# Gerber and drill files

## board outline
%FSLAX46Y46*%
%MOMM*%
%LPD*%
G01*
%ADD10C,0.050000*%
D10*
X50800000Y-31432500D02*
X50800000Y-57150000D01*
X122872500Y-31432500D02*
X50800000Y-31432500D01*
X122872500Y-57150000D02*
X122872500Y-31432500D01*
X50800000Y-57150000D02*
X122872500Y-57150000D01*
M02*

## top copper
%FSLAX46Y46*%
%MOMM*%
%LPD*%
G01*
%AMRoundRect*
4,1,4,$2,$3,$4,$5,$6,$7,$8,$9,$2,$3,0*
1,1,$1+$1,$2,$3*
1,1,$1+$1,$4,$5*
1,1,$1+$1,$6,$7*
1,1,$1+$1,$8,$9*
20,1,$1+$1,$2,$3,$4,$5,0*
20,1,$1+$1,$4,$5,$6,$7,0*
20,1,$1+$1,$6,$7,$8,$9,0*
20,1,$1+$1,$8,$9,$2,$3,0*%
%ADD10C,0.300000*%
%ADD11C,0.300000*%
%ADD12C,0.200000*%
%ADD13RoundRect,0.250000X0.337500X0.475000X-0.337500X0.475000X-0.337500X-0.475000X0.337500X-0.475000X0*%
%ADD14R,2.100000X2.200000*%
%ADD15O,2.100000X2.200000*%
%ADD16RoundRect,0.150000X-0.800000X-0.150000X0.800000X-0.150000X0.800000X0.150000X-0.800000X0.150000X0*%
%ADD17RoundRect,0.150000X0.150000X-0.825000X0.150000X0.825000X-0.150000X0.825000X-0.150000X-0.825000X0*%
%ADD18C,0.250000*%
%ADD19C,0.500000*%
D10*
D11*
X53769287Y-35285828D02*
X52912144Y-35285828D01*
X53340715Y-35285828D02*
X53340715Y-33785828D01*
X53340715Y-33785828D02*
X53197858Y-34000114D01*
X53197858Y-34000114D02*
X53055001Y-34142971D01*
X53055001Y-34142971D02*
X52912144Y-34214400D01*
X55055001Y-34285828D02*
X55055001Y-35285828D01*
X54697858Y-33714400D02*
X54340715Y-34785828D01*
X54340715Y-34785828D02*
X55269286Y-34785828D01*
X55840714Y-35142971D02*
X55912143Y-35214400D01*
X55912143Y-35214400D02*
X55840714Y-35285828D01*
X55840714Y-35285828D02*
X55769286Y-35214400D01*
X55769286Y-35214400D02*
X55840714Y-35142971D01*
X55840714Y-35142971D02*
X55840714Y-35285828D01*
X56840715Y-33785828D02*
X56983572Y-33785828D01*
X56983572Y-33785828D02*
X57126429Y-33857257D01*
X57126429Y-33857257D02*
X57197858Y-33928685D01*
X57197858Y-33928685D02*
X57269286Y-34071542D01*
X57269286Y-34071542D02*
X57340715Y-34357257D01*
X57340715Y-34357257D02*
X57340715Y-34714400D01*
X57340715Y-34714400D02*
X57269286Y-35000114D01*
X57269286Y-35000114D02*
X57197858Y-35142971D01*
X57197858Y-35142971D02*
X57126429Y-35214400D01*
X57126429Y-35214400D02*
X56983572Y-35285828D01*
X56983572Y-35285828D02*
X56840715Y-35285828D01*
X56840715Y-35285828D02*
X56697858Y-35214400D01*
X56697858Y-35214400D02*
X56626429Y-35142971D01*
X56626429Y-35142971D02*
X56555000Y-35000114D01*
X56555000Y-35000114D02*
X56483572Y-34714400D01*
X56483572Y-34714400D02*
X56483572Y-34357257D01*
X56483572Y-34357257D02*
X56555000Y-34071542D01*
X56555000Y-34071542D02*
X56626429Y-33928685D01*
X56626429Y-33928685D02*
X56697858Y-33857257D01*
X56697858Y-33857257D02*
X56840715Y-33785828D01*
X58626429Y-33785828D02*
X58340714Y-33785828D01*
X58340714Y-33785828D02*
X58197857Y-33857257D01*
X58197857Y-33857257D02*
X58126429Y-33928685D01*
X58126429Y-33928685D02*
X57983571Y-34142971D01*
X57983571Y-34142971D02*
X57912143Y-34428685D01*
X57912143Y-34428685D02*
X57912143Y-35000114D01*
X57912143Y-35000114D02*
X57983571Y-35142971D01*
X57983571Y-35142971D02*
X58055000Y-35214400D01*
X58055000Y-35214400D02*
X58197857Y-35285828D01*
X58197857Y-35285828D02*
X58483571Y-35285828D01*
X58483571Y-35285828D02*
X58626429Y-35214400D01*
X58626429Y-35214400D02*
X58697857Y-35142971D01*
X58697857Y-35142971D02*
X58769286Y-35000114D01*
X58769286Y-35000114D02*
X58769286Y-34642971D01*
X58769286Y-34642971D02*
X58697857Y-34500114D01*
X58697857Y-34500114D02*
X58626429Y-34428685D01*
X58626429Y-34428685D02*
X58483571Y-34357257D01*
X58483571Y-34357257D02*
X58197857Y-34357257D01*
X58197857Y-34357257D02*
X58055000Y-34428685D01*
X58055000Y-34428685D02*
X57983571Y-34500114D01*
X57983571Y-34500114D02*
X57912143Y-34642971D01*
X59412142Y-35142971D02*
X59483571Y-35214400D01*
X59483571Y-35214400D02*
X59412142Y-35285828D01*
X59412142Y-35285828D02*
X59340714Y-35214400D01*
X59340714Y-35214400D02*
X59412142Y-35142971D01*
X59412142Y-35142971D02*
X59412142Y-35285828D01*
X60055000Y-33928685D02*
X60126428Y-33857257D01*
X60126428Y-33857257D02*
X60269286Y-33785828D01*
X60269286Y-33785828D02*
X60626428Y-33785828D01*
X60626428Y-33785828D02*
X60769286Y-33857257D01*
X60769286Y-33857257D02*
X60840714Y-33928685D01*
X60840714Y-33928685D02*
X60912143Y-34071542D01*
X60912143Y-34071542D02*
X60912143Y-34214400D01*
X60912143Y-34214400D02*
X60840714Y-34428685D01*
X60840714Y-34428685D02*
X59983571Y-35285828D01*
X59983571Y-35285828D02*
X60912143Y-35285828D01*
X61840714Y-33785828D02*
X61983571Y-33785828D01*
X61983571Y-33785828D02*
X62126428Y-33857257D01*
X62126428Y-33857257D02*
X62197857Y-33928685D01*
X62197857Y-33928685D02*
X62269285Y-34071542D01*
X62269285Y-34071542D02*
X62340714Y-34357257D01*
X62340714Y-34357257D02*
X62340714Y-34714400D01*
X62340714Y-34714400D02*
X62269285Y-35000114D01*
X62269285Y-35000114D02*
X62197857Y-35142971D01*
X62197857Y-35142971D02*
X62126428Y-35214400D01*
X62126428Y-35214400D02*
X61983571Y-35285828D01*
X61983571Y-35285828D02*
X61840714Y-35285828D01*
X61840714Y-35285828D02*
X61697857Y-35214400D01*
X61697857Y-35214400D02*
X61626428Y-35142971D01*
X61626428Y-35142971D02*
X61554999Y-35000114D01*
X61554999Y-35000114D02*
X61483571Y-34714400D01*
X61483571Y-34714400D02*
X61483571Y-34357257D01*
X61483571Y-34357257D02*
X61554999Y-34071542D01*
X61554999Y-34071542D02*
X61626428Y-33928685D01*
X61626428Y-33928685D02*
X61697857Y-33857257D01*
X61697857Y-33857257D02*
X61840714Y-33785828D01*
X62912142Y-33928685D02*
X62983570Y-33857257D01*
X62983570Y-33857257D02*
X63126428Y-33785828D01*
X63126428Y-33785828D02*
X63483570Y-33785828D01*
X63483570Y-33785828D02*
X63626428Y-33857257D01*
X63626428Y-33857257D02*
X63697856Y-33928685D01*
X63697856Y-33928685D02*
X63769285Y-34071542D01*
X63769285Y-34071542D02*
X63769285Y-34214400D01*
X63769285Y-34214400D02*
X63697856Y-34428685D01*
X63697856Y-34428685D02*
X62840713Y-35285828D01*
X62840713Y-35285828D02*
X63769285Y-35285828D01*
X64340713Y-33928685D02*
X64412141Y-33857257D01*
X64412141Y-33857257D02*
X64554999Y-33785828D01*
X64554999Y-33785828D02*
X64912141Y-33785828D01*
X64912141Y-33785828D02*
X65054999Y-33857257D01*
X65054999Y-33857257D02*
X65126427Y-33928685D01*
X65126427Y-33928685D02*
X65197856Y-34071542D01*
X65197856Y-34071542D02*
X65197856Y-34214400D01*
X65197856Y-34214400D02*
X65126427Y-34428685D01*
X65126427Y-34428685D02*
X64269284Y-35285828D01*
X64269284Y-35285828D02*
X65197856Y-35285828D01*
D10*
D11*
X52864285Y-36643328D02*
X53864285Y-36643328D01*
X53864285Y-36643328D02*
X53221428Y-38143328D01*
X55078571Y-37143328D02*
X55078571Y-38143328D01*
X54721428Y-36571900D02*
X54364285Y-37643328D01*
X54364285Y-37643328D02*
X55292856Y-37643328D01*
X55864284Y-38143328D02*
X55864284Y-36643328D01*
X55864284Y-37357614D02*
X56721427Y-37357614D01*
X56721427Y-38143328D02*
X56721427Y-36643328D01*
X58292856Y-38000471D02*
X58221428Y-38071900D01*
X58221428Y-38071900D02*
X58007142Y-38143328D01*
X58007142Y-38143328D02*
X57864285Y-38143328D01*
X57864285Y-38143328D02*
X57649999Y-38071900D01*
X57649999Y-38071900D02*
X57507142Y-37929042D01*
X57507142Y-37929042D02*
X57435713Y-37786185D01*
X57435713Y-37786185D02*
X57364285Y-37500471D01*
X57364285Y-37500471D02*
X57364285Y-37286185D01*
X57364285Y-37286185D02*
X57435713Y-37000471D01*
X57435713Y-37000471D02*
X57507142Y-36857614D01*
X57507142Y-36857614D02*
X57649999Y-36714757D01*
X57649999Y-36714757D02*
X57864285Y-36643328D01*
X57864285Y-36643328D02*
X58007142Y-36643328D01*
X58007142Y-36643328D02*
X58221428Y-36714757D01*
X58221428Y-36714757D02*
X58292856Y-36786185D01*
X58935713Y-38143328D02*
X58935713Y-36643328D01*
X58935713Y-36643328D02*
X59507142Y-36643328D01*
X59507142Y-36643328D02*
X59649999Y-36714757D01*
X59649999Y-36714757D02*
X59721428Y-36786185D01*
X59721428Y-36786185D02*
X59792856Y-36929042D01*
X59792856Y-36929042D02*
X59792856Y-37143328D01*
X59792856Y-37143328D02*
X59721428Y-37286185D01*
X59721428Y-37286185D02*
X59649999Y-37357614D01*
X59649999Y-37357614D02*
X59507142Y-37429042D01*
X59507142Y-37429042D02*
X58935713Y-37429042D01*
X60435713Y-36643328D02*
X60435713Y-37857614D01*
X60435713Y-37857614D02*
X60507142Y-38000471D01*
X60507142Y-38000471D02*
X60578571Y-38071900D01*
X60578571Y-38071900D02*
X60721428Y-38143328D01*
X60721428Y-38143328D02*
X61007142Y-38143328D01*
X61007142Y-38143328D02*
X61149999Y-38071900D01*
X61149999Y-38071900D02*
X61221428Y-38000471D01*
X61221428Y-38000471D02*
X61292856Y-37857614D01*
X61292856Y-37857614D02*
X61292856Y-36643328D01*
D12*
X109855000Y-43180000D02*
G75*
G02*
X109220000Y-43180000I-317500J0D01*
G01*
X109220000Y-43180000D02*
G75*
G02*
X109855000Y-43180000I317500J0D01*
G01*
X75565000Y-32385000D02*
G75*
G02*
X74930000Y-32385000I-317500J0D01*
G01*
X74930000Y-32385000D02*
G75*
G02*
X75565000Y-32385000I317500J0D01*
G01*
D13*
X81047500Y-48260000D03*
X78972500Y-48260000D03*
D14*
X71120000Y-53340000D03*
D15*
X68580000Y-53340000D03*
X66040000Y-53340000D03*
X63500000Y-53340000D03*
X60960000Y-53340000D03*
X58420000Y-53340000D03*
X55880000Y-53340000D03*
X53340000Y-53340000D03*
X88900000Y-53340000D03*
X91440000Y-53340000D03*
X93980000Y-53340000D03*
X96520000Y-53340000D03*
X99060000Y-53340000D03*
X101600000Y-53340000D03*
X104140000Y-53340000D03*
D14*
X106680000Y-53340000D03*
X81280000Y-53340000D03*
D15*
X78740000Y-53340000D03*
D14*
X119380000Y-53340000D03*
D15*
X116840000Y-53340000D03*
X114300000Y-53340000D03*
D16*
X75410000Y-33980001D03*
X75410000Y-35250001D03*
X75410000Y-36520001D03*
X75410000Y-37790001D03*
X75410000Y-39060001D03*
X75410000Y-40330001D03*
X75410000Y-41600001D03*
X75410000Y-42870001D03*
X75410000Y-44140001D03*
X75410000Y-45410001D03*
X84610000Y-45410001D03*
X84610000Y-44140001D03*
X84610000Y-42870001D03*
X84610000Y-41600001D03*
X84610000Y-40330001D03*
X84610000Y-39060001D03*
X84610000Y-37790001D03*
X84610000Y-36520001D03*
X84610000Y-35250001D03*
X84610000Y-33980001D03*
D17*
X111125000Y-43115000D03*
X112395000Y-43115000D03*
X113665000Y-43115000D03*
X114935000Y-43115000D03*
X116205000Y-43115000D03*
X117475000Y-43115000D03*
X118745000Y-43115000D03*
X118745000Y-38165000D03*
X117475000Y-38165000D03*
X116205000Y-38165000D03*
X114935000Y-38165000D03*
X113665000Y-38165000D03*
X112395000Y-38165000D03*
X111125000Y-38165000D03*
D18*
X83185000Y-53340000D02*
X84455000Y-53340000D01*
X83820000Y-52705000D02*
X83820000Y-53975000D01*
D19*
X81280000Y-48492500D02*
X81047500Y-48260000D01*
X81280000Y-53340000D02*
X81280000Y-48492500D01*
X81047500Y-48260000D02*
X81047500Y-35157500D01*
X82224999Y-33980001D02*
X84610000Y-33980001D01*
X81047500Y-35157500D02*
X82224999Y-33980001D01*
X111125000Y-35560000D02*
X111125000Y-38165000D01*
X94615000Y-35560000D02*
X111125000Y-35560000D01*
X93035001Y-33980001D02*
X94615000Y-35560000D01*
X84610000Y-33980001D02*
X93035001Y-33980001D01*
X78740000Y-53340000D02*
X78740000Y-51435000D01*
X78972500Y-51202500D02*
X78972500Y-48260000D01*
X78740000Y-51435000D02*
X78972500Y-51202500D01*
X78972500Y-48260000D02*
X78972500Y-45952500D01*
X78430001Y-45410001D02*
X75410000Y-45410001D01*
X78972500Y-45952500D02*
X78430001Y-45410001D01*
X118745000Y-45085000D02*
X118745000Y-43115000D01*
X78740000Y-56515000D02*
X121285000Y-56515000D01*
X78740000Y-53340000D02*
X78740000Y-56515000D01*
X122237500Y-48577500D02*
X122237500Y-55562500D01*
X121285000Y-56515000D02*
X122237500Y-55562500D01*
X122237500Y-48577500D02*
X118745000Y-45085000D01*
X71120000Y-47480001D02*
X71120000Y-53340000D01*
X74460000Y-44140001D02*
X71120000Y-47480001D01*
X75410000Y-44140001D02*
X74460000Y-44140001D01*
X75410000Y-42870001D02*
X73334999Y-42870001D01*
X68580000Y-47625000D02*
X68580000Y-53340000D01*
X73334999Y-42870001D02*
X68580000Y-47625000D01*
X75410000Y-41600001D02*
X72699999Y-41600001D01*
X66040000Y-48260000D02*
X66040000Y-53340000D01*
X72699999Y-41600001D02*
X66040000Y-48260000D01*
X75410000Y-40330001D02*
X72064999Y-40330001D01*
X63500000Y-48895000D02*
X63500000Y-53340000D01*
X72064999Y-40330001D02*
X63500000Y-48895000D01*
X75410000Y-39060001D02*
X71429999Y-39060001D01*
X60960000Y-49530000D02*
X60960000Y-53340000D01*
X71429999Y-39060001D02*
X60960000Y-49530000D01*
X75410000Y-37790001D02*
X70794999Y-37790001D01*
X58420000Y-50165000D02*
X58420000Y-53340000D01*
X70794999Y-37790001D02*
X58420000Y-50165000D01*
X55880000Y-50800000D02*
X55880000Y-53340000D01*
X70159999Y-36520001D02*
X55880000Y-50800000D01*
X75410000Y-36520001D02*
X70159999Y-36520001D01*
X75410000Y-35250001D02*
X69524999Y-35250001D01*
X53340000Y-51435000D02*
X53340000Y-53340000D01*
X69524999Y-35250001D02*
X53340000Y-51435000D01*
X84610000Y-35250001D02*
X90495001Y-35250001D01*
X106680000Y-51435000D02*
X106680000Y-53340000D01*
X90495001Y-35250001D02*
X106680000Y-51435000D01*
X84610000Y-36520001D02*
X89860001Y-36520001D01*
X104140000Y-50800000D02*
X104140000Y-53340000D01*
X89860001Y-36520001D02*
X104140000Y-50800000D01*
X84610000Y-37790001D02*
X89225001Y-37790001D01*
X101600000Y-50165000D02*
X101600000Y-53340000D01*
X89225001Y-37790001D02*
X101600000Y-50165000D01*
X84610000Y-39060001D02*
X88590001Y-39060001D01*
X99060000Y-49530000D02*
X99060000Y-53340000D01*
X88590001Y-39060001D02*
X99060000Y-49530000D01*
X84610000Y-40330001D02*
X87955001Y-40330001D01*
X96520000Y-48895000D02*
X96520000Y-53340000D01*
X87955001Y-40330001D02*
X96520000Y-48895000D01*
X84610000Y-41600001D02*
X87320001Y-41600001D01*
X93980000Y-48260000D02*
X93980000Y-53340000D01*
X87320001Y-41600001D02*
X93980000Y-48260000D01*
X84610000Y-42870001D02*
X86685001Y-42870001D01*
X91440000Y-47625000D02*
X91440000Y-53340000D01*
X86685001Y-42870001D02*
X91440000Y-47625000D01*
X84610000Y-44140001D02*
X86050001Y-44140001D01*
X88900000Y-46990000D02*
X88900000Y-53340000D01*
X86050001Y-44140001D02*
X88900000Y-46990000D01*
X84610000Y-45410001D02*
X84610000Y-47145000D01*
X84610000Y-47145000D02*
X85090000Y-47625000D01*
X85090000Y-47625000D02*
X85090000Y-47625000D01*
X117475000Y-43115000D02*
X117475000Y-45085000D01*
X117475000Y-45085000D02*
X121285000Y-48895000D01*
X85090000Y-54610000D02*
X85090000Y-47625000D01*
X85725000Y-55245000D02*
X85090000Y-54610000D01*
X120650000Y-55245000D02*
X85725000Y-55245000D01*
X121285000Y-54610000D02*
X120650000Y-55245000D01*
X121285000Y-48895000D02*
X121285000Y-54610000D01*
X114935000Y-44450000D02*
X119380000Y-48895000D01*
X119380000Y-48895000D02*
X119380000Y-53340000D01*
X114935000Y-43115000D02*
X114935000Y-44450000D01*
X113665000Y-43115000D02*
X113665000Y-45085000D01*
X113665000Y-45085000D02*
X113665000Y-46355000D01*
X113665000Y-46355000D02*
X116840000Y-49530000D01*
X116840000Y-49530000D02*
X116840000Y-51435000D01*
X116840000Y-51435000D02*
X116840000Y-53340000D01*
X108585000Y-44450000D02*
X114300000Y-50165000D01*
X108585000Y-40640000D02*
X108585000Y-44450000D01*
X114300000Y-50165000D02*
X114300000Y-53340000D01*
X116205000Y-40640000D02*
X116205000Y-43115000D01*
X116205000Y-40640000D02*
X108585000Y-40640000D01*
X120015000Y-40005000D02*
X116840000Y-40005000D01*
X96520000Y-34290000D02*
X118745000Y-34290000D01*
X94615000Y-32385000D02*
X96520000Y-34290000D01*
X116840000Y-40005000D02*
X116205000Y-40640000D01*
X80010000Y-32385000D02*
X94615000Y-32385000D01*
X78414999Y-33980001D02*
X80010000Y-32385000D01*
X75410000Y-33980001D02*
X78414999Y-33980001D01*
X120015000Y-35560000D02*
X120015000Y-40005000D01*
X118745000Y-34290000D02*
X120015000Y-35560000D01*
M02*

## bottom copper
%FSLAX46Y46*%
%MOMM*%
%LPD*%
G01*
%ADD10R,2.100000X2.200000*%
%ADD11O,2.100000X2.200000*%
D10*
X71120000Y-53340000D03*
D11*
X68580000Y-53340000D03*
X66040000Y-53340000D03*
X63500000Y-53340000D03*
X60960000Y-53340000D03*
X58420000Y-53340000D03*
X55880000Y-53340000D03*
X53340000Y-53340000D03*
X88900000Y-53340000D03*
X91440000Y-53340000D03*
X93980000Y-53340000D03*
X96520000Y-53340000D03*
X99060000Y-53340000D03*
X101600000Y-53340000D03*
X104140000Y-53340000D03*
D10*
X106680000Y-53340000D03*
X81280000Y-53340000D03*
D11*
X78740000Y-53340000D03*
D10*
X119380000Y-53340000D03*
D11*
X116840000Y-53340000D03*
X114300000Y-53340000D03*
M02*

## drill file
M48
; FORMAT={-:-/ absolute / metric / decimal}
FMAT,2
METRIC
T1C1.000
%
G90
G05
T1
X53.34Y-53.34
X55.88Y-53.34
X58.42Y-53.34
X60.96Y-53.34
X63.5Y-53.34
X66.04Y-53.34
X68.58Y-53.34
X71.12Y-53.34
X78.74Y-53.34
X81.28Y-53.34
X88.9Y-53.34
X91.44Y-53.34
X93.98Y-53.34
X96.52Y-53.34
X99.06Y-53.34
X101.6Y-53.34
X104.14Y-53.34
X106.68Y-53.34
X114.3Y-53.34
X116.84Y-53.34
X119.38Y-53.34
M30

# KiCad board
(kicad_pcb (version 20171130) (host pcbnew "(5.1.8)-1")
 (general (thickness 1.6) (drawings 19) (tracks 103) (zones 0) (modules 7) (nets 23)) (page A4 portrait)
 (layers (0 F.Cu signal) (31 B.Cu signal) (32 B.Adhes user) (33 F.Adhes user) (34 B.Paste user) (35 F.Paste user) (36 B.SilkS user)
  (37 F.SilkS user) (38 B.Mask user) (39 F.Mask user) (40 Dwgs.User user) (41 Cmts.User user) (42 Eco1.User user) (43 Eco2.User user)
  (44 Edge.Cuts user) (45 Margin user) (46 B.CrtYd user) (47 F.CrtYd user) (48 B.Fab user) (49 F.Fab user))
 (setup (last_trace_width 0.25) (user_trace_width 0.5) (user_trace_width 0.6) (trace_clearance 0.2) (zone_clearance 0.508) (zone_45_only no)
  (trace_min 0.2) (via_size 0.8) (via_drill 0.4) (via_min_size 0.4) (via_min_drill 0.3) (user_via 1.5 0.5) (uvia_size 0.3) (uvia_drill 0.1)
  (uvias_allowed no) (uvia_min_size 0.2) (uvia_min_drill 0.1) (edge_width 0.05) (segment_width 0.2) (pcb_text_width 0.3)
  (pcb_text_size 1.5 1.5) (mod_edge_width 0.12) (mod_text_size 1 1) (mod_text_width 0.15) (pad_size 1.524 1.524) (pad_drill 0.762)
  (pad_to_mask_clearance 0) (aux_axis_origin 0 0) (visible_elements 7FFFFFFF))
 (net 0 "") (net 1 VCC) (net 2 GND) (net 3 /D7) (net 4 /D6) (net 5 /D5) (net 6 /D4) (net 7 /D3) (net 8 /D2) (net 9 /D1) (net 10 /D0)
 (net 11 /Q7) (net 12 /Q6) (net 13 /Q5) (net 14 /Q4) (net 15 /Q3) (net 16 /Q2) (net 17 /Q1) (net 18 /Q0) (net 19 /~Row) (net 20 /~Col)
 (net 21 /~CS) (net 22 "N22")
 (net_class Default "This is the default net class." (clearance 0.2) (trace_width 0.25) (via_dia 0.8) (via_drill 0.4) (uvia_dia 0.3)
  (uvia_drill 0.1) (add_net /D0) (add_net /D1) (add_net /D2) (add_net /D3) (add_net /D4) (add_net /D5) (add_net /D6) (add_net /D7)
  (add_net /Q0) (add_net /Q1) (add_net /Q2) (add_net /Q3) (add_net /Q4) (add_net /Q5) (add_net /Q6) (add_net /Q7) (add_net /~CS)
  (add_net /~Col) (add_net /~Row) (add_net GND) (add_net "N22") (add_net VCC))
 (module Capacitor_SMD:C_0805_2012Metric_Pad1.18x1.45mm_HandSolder (layer F.Cu) (at 80.01 48.26 180)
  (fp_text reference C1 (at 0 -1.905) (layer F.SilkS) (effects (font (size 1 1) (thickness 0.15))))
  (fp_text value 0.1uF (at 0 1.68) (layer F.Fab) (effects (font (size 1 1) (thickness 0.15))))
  (pad 1 smd roundrect (at -1.0375 0 180) (size 1.175 1.45) (layers F.Cu F.Paste F.Mask) (roundrect_rratio 0.2127659574468085) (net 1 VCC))
  (pad 2 smd roundrect (at 1.0375 0 180) (size 1.175 1.45) (layers F.Cu F.Paste F.Mask) (roundrect_rratio 0.2127659574468085) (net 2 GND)))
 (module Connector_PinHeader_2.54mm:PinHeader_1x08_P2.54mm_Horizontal (layer F.Cu) (at 71.12 53.34 270)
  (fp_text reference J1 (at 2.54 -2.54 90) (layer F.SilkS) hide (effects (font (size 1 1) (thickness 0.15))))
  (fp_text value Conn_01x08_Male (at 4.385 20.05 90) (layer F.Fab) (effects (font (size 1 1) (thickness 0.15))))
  (pad 1 thru_hole rect (at 0 0 270) (size 2.2 2.1) (drill 1) (layers *.Cu *.Mask) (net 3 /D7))
  (pad 2 thru_hole oval (at 0 2.54 270) (size 2.2 2.1) (drill 1) (layers *.Cu *.Mask) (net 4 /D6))
  (pad 3 thru_hole oval (at 0 5.08 270) (size 2.2 2.1) (drill 1) (layers *.Cu *.Mask) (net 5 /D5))
  (pad 4 thru_hole oval (at 0 7.62 270) (size 2.2 2.1) (drill 1) (layers *.Cu *.Mask) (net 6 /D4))
  (pad 5 thru_hole oval (at 0 10.16 270) (size 2.2 2.1) (drill 1) (layers *.Cu *.Mask) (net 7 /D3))
  (pad 6 thru_hole oval (at 0 12.7 270) (size 2.2 2.1) (drill 1) (layers *.Cu *.Mask) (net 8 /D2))
  (pad 7 thru_hole oval (at 0 15.24 270) (size 2.2 2.1) (drill 1) (layers *.Cu *.Mask) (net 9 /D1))
  (pad 8 thru_hole oval (at 0 17.78 270) (size 2.2 2.1) (drill 1) (layers *.Cu *.Mask) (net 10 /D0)))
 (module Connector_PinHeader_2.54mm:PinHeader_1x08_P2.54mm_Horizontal (layer F.Cu) (at 106.68 53.34 270)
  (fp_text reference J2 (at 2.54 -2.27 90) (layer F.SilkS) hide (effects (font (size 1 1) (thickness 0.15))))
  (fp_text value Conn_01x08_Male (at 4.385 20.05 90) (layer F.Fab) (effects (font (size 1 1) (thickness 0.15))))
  (pad 8 thru_hole oval (at 0 17.78 270) (size 2.2 2.1) (drill 1) (layers *.Cu *.Mask) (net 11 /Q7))
  (pad 7 thru_hole oval (at 0 15.24 270) (size 2.2 2.1) (drill 1) (layers *.Cu *.Mask) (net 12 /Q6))
  (pad 6 thru_hole oval (at 0 12.7 270) (size 2.2 2.1) (drill 1) (layers *.Cu *.Mask) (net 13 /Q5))
  (pad 5 thru_hole oval (at 0 10.16 270) (size 2.2 2.1) (drill 1) (layers *.Cu *.Mask) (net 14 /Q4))
  (pad 4 thru_hole oval (at 0 7.62 270) (size 2.2 2.1) (drill 1) (layers *.Cu *.Mask) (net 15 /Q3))
  (pad 3 thru_hole oval (at 0 5.08 270) (size 2.2 2.1) (drill 1) (layers *.Cu *.Mask) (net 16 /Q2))
  (pad 2 thru_hole oval (at 0 2.54 270) (size 2.2 2.1) (drill 1) (layers *.Cu *.Mask) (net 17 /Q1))
  (pad 1 thru_hole rect (at 0 0 270) (size 2.2 2.1) (drill 1) (layers *.Cu *.Mask) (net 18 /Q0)))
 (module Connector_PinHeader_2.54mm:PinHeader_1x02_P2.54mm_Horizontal (layer F.Cu) (at 81.28 53.34 270)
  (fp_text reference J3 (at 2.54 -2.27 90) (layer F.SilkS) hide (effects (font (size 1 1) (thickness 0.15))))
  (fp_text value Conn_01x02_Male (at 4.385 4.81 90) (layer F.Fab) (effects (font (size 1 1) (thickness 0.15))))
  (pad 1 thru_hole rect (at 0 0 270) (size 2.2 2.1) (drill 1) (layers *.Cu *.Mask) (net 1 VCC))
  (pad 2 thru_hole oval (at 0 2.54 270) (size 2.2 2.1) (drill 1) (layers *.Cu *.Mask) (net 2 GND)))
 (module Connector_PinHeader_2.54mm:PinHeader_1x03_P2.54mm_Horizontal (layer F.Cu) (at 119.38 53.34 270)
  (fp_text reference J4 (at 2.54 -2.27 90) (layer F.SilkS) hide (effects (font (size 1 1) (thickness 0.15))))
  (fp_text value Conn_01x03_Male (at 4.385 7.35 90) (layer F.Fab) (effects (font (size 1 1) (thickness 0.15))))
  (pad 1 thru_hole rect (at 0 0 270) (size 2.2 2.1) (drill 1) (layers *.Cu *.Mask) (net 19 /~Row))
  (pad 2 thru_hole oval (at 0 2.54 270) (size 2.2 2.1) (drill 1) (layers *.Cu *.Mask) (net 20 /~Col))
  (pad 3 thru_hole oval (at 0 5.08 270) (size 2.2 2.1) (drill 1) (layers *.Cu *.Mask) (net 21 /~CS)))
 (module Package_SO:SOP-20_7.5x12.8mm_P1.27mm (layer F.Cu) (at 80.01 39.695001)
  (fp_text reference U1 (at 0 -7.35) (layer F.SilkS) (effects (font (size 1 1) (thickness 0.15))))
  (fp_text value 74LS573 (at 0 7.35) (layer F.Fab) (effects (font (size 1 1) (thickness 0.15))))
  (pad 1 smd roundrect (at -4.6 -5.715) (size 1.9 0.6) (layers F.Cu F.Paste F.Mask) (roundrect_rratio 0.25) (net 21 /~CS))
  (pad 2 smd roundrect (at -4.6 -4.445) (size 1.9 0.6) (layers F.Cu F.Paste F.Mask) (roundrect_rratio 0.25) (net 10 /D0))
  (pad 3 smd roundrect (at -4.6 -3.175) (size 1.9 0.6) (layers F.Cu F.Paste F.Mask) (roundrect_rratio 0.25) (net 9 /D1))
  (pad 4 smd roundrect (at -4.6 -1.905) (size 1.9 0.6) (layers F.Cu F.Paste F.Mask) (roundrect_rratio 0.25) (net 8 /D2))
  (pad 5 smd roundrect (at -4.6 -0.635) (size 1.9 0.6) (layers F.Cu F.Paste F.Mask) (roundrect_rratio 0.25) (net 7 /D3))
  (pad 6 smd roundrect (at -4.6 0.635) (size 1.9 0.6) (layers F.Cu F.Paste F.Mask) (roundrect_rratio 0.25) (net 6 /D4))
  (pad 7 smd roundrect (at -4.6 1.905) (size 1.9 0.6) (layers F.Cu F.Paste F.Mask) (roundrect_rratio 0.25) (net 5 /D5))
  (pad 8 smd roundrect (at -4.6 3.175) (size 1.9 0.6) (layers F.Cu F.Paste F.Mask) (roundrect_rratio 0.25) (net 4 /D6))
  (pad 9 smd roundrect (at -4.6 4.445) (size 1.9 0.6) (layers F.Cu F.Paste F.Mask) (roundrect_rratio 0.25) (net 3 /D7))
  (pad 10 smd roundrect (at -4.6 5.715) (size 1.9 0.6) (layers F.Cu F.Paste F.Mask) (roundrect_rratio 0.25) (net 2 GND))
  (pad 11 smd roundrect (at 4.6 5.715) (size 1.9 0.6) (layers F.Cu F.Paste F.Mask) (roundrect_rratio 0.25) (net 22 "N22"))
  (pad 12 smd roundrect (at 4.6 4.445) (size 1.9 0.6) (layers F.Cu F.Paste F.Mask) (roundrect_rratio 0.25) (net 11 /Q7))
  (pad 13 smd roundrect (at 4.6 3.175) (size 1.9 0.6) (layers F.Cu F.Paste F.Mask) (roundrect_rratio 0.25) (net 12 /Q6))
  (pad 14 smd roundrect (at 4.6 1.905) (size 1.9 0.6) (layers F.Cu F.Paste F.Mask) (roundrect_rratio 0.25) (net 13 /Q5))
  (pad 15 smd roundrect (at 4.6 0.635) (size 1.9 0.6) (layers F.Cu F.Paste F.Mask) (roundrect_rratio 0.25) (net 14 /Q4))
  (pad 16 smd roundrect (at 4.6 -0.635) (size 1.9 0.6) (layers F.Cu F.Paste F.Mask) (roundrect_rratio 0.25) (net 15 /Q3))
  (pad 17 smd roundrect (at 4.6 -1.905) (size 1.9 0.6) (layers F.Cu F.Paste F.Mask) (roundrect_rratio 0.25) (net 16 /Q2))
  (pad 18 smd roundrect (at 4.6 -3.175) (size 1.9 0.6) (layers F.Cu F.Paste F.Mask) (roundrect_rratio 0.25) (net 17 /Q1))
  (pad 19 smd roundrect (at 4.6 -4.445) (size 1.9 0.6) (layers F.Cu F.Paste F.Mask) (roundrect_rratio 0.25) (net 18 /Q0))
  (pad 20 smd roundrect (at 4.6 -5.715) (size 1.9 0.6) (layers F.Cu F.Paste F.Mask) (roundrect_rratio 0.25) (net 1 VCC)))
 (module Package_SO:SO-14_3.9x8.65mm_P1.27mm (layer F.Cu) (at 114.935 40.64 90)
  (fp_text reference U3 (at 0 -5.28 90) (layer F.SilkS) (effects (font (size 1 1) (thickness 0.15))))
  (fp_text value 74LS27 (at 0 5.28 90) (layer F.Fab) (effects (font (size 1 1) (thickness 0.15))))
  (pad 1 smd roundrect (at -2.475 -3.81 90) (size 1.95 0.6) (layers F.Cu F.Paste F.Mask) (roundrect_rratio 0.25))
  (pad 2 smd roundrect (at -2.475 -2.54 90) (size 1.95 0.6) (layers F.Cu F.Paste F.Mask) (roundrect_rratio 0.25))
  (pad 3 smd roundrect (at -2.475 -1.27 90) (size 1.95 0.6) (layers F.Cu F.Paste F.Mask) (roundrect_rratio 0.25) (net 20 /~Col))
  (pad 4 smd roundrect (at -2.475 0 90) (size 1.95 0.6) (layers F.Cu F.Paste F.Mask) (roundrect_rratio 0.25) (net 19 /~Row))
  (pad 5 smd roundrect (at -2.475 1.27 90) (size 1.95 0.6) (layers F.Cu F.Paste F.Mask) (roundrect_rratio 0.25) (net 21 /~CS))
  (pad 6 smd roundrect (at -2.475 2.54 90) (size 1.95 0.6) (layers F.Cu F.Paste F.Mask) (roundrect_rratio 0.25) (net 22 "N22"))
  (pad 7 smd roundrect (at -2.475 3.81 90) (size 1.95 0.6) (layers F.Cu F.Paste F.Mask) (roundrect_rratio 0.25) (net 2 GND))
  (pad 8 smd roundrect (at 2.475 3.81 90) (size 1.95 0.6) (layers F.Cu F.Paste F.Mask) (roundrect_rratio 0.25))
  (pad 9 smd roundrect (at 2.475 2.54 90) (size 1.95 0.6) (layers F.Cu F.Paste F.Mask) (roundrect_rratio 0.25))
  (pad 10 smd roundrect (at 2.475 1.27 90) (size 1.95 0.6) (layers F.Cu F.Paste F.Mask) (roundrect_rratio 0.25))
  (pad 11 smd roundrect (at 2.475 0 90) (size 1.95 0.6) (layers F.Cu F.Paste F.Mask) (roundrect_rratio 0.25))
  (pad 12 smd roundrect (at 2.475 -1.27 90) (size 1.95 0.6) (layers F.Cu F.Paste F.Mask) (roundrect_rratio 0.25))
  (pad 13 smd roundrect (at 2.475 -2.54 90) (size 1.95 0.6) (layers F.Cu F.Paste F.Mask) (roundrect_rratio 0.25))
  (pad 14 smd roundrect (at 2.475 -3.81 90) (size 1.95 0.6) (layers F.Cu F.Paste F.Mask) (roundrect_rratio 0.25) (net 1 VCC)))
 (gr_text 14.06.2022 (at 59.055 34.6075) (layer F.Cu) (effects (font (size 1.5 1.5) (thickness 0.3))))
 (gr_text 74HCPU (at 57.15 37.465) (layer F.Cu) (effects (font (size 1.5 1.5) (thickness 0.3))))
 (gr_circle (center 109.5375 43.18) (end 109.855 43.18) (layer F.Cu) (width 0.2))
 (gr_circle (center 75.2475 32.385) (end 75.565 32.385) (layer F.Cu) (width 0.2))
 (gr_line (start 50.8 31.4325) (end 50.8 57.15) (layer Edge.Cuts) (width 0.05))
 (gr_line (start 122.8725 31.4325) (end 50.8 31.4325) (layer Edge.Cuts) (width 0.05))
 (gr_line (start 122.8725 57.15) (end 122.8725 31.4325) (layer Edge.Cuts) (width 0.05))
 (gr_line (start 50.8 57.15) (end 122.8725 57.15) (layer Edge.Cuts) (width 0.05))
 (segment (start 83.185 53.34) (end 84.455 53.34) (width 0.25) (layer F.Cu) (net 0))
 (segment (start 83.82 52.705) (end 83.82 53.975) (width 0.25) (layer F.Cu) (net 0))
 (segment (start 81.28 48.4925) (end 81.0475 48.26) (width 0.5) (layer F.Cu) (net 1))
 (segment (start 81.28 53.34) (end 81.28 48.4925) (width 0.5) (layer F.Cu) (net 1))
 (segment (start 81.0475 48.26) (end 81.0475 35.1575) (width 0.5) (layer F.Cu) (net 1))
 (segment (start 82.224999 33.980001) (end 84.61 33.980001) (width 0.5) (layer F.Cu) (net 1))
 (segment (start 81.0475 35.1575) (end 82.224999 33.980001) (width 0.5) (layer F.Cu) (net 1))
 (segment (start 111.125 35.56) (end 111.125 38.165) (width 0.5) (layer F.Cu) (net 1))
 (segment (start 94.615 35.56) (end 111.125 35.56) (width 0.5) (layer F.Cu) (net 1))
 (segment (start 93.035001 33.980001) (end 94.615 35.56) (width 0.5) (layer F.Cu) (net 1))
 (segment (start 84.61 33.980001) (end 93.035001 33.980001) (width 0.5) (layer F.Cu) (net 1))
 (segment (start 78.74 53.34) (end 78.74 51.435) (width 0.5) (layer F.Cu) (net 2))
 (segment (start 78.9725 51.2025) (end 78.9725 48.26) (width 0.5) (layer F.Cu) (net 2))
 (segment (start 78.74 51.435) (end 78.9725 51.2025) (width 0.5) (layer F.Cu) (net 2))
 (segment (start 78.9725 48.26) (end 78.9725 45.9525) (width 0.5) (layer F.Cu) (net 2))
 (segment (start 78.430001 45.410001) (end 75.41 45.410001) (width 0.5) (layer F.Cu) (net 2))
 (segment (start 78.9725 45.9525) (end 78.430001 45.410001) (width 0.5) (layer F.Cu) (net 2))
 (segment (start 118.745 45.085) (end 118.745 43.115) (width 0.5) (layer F.Cu) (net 2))
 (segment (start 78.74 56.515) (end 121.285 56.515) (width 0.5) (layer F.Cu) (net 2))
 (segment (start 78.74 53.34) (end 78.74 56.515) (width 0.5) (layer F.Cu) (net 2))
 (segment (start 122.2375 48.5775) (end 122.2375 55.5625) (width 0.5) (layer F.Cu) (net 2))
 (segment (start 121.285 56.515) (end 122.2375 55.5625) (width 0.5) (layer F.Cu) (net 2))
 (segment (start 122.2375 48.5775) (end 118.745 45.085) (width 0.5) (layer F.Cu) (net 2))
 (segment (start 71.12 47.480001) (end 71.12 53.34) (width 0.5) (layer F.Cu) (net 3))
 (segment (start 74.46 44.140001) (end 71.12 47.480001) (width 0.5) (layer F.Cu) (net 3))
 (segment (start 75.41 44.140001) (end 74.46 44.140001) (width 0.5) (layer F.Cu) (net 3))
 (segment (start 75.41 42.870001) (end 73.334999 42.870001) (width 0.5) (layer F.Cu) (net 4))
 (segment (start 68.58 47.625) (end 68.58 53.34) (width 0.5) (layer F.Cu) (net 4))
 (segment (start 73.334999 42.870001) (end 68.58 47.625) (width 0.5) (layer F.Cu) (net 4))
 (segment (start 75.41 41.600001) (end 72.699999 41.600001) (width 0.5) (layer F.Cu) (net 5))
 (segment (start 66.04 48.26) (end 66.04 53.34) (width 0.5) (layer F.Cu) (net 5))
 (segment (start 72.699999 41.600001) (end 66.04 48.26) (width 0.5) (layer F.Cu) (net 5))
 (segment (start 75.41 40.330001) (end 72.064999 40.330001) (width 0.5) (layer F.Cu) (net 6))
 (segment (start 63.5 48.895) (end 63.5 53.34) (width 0.5) (layer F.Cu) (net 6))
 (segment (start 72.064999 40.330001) (end 63.5 48.895) (width 0.5) (layer F.Cu) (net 6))
 (segment (start 75.41 39.060001) (end 71.429999 39.060001) (width 0.5) (layer F.Cu) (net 7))
 (segment (start 60.96 49.53) (end 60.96 53.34) (width 0.5) (layer F.Cu) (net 7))
 (segment (start 71.429999 39.060001) (end 60.96 49.53) (width 0.5) (layer F.Cu) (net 7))
 (segment (start 75.41 37.790001) (end 70.794999 37.790001) (width 0.5) (layer F.Cu) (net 8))
 (segment (start 58.42 50.165) (end 58.42 53.34) (width 0.5) (layer F.Cu) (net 8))
 (segment (start 70.794999 37.790001) (end 58.42 50.165) (width 0.5) (layer F.Cu) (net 8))
 (segment (start 55.88 50.8) (end 55.88 53.34) (width 0.5) (layer F.Cu) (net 9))
 (segment (start 70.159999 36.520001) (end 55.88 50.8) (width 0.5) (layer F.Cu) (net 9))
 (segment (start 75.41 36.520001) (end 70.159999 36.520001) (width 0.5) (layer F.Cu) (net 9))
 (segment (start 75.41 35.250001) (end 69.524999 35.250001) (width 0.5) (layer F.Cu) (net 10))
 (segment (start 53.34 51.435) (end 53.34 53.34) (width 0.5) (layer F.Cu) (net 10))
 (segment (start 69.524999 35.250001) (end 53.34 51.435) (width 0.5) (layer F.Cu) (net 10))
 (segment (start 84.61 35.250001) (end 90.495001 35.250001) (width 0.5) (layer F.Cu) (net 18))
 (segment (start 106.68 51.435) (end 106.68 53.34) (width 0.5) (layer F.Cu) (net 18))
 (segment (start 90.495001 35.250001) (end 106.68 51.435) (width 0.5) (layer F.Cu) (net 18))
 (segment (start 84.61 36.520001) (end 89.860001 36.520001) (width 0.5) (layer F.Cu) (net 17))
 (segment (start 104.14 50.8) (end 104.14 53.34) (width 0.5) (layer F.Cu) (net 17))
 (segment (start 89.860001 36.520001) (end 104.14 50.8) (width 0.5) (layer F.Cu) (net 17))
 (segment (start 84.61 37.790001) (end 89.225001 37.790001) (width 0.5) (layer F.Cu) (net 16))
 (segment (start 101.6 50.165) (end 101.6 53.34) (width 0.5) (layer F.Cu) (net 16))
 (segment (start 89.225001 37.790001) (end 101.6 50.165) (width 0.5) (layer F.Cu) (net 16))
 (segment (start 84.61 39.060001) (end 88.590001 39.060001) (width 0.5) (layer F.Cu) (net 15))
 (segment (start 99.06 49.53) (end 99.06 53.34) (width 0.5) (layer F.Cu) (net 15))
 (segment (start 88.590001 39.060001) (end 99.06 49.53) (width 0.5) (layer F.Cu) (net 15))
 (segment (start 84.61 40.330001) (end 87.955001 40.330001) (width 0.5) (layer F.Cu) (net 14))
 (segment (start 96.52 48.895) (end 96.52 53.34) (width 0.5) (layer F.Cu) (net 14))
 (segment (start 87.955001 40.330001) (end 96.52 48.895) (width 0.5) (layer F.Cu) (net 14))
 (segment (start 84.61 41.600001) (end 87.320001 41.600001) (width 0.5) (layer F.Cu) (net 13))
 (segment (start 93.98 48.26) (end 93.98 53.34) (width 0.5) (layer F.Cu) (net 13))
 (segment (start 87.320001 41.600001) (end 93.98 48.26) (width 0.5) (layer F.Cu) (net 13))
 (segment (start 84.61 42.870001) (end 86.685001 42.870001) (width 0.5) (layer F.Cu) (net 12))
 (segment (start 91.44 47.625) (end 91.44 53.34) (width 0.5) (layer F.Cu) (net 12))
 (segment (start 86.685001 42.870001) (end 91.44 47.625) (width 0.5) (layer F.Cu) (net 12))
 (segment (start 84.61 44.140001) (end 86.050001 44.140001) (width 0.5) (layer F.Cu) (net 11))
 (segment (start 88.9 46.99) (end 88.9 53.34) (width 0.5) (layer F.Cu) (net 11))
 (segment (start 86.050001 44.140001) (end 88.9 46.99) (width 0.5) (layer F.Cu) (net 11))
 (segment (start 84.61 45.410001) (end 84.61 47.145) (width 0.5) (layer F.Cu) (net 22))
 (segment (start 84.61 47.145) (end 85.09 47.625) (width 0.5) (layer F.Cu) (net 22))
 (segment (start 85.09 47.625) (end 85.09 47.625) (width 0.5) (layer F.Cu) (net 22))
 (segment (start 117.475 43.115) (end 117.475 45.085) (width 0.5) (layer F.Cu) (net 22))
 (segment (start 117.475 45.085) (end 121.285 48.895) (width 0.5) (layer F.Cu) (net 22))
 (segment (start 85.09 54.61) (end 85.09 47.625) (width 0.5) (layer F.Cu) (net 22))
 (segment (start 85.725 55.245) (end 85.09 54.61) (width 0.5) (layer F.Cu) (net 22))
 (segment (start 120.65 55.245) (end 85.725 55.245) (width 0.5) (layer F.Cu) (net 22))
 (segment (start 121.285 54.61) (end 120.65 55.245) (width 0.5) (layer F.Cu) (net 22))
 (segment (start 121.285 48.895) (end 121.285 54.61) (width 0.5) (layer F.Cu) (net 22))
 (segment (start 114.935 44.45) (end 119.38 48.895) (width 0.5) (layer F.Cu) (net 19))
 (segment (start 119.38 48.895) (end 119.38 53.34) (width 0.5) (layer F.Cu) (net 19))
 (segment (start 114.935 43.115) (end 114.935 44.45) (width 0.5) (layer F.Cu) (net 19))
 (segment (start 113.665 43.115) (end 113.665 45.085) (width 0.5) (layer F.Cu) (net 20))
 (segment (start 113.665 45.085) (end 113.665 46.355) (width 0.5) (layer F.Cu) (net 20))
 (segment (start 113.665 46.355) (end 116.84 49.53) (width 0.5) (layer F.Cu) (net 20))
 (segment (start 116.84 49.53) (end 116.84 51.435) (width 0.5) (layer F.Cu) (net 20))
 (segment (start 116.84 51.435) (end 116.84 53.34) (width 0.5) (layer F.Cu) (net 20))
 (segment (start 108.585 44.45) (end 114.3 50.165) (width 0.5) (layer F.Cu) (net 21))
 (segment (start 108.585 40.64) (end 108.585 44.45) (width 0.5) (layer F.Cu) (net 21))
 (segment (start 114.3 50.165) (end 114.3 53.34) (width 0.5) (layer F.Cu) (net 21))
 (segment (start 116.205 40.64) (end 116.205 43.115) (width 0.5) (layer F.Cu) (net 21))
 (segment (start 116.205 40.64) (end 108.585 40.64) (width 0.5) (layer F.Cu) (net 21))
 (segment (start 120.015 40.005) (end 116.84 40.005) (width 0.5) (layer F.Cu) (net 21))
 (segment (start 96.52 34.29) (end 118.745 34.29) (width 0.5) (layer F.Cu) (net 21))
 (segment (start 94.615 32.385) (end 96.52 34.29) (width 0.5) (layer F.Cu) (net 21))
 (segment (start 116.84 40.005) (end 116.205 40.64) (width 0.5) (layer F.Cu) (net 21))
 (segment (start 80.01 32.385) (end 94.615 32.385) (width 0.5) (layer F.Cu) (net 21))
 (segment (start 78.414999 33.980001) (end 80.01 32.385) (width 0.5) (layer F.Cu) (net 21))
 (segment (start 75.41 33.980001) (end 78.414999 33.980001) (width 0.5) (layer F.Cu) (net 21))
 (segment (start 120.015 35.56) (end 120.015 40.005) (width 0.5) (layer F.Cu) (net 21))
 (segment (start 118.745 34.29) (end 120.015 35.56) (width 0.5) (layer F.Cu) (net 21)))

